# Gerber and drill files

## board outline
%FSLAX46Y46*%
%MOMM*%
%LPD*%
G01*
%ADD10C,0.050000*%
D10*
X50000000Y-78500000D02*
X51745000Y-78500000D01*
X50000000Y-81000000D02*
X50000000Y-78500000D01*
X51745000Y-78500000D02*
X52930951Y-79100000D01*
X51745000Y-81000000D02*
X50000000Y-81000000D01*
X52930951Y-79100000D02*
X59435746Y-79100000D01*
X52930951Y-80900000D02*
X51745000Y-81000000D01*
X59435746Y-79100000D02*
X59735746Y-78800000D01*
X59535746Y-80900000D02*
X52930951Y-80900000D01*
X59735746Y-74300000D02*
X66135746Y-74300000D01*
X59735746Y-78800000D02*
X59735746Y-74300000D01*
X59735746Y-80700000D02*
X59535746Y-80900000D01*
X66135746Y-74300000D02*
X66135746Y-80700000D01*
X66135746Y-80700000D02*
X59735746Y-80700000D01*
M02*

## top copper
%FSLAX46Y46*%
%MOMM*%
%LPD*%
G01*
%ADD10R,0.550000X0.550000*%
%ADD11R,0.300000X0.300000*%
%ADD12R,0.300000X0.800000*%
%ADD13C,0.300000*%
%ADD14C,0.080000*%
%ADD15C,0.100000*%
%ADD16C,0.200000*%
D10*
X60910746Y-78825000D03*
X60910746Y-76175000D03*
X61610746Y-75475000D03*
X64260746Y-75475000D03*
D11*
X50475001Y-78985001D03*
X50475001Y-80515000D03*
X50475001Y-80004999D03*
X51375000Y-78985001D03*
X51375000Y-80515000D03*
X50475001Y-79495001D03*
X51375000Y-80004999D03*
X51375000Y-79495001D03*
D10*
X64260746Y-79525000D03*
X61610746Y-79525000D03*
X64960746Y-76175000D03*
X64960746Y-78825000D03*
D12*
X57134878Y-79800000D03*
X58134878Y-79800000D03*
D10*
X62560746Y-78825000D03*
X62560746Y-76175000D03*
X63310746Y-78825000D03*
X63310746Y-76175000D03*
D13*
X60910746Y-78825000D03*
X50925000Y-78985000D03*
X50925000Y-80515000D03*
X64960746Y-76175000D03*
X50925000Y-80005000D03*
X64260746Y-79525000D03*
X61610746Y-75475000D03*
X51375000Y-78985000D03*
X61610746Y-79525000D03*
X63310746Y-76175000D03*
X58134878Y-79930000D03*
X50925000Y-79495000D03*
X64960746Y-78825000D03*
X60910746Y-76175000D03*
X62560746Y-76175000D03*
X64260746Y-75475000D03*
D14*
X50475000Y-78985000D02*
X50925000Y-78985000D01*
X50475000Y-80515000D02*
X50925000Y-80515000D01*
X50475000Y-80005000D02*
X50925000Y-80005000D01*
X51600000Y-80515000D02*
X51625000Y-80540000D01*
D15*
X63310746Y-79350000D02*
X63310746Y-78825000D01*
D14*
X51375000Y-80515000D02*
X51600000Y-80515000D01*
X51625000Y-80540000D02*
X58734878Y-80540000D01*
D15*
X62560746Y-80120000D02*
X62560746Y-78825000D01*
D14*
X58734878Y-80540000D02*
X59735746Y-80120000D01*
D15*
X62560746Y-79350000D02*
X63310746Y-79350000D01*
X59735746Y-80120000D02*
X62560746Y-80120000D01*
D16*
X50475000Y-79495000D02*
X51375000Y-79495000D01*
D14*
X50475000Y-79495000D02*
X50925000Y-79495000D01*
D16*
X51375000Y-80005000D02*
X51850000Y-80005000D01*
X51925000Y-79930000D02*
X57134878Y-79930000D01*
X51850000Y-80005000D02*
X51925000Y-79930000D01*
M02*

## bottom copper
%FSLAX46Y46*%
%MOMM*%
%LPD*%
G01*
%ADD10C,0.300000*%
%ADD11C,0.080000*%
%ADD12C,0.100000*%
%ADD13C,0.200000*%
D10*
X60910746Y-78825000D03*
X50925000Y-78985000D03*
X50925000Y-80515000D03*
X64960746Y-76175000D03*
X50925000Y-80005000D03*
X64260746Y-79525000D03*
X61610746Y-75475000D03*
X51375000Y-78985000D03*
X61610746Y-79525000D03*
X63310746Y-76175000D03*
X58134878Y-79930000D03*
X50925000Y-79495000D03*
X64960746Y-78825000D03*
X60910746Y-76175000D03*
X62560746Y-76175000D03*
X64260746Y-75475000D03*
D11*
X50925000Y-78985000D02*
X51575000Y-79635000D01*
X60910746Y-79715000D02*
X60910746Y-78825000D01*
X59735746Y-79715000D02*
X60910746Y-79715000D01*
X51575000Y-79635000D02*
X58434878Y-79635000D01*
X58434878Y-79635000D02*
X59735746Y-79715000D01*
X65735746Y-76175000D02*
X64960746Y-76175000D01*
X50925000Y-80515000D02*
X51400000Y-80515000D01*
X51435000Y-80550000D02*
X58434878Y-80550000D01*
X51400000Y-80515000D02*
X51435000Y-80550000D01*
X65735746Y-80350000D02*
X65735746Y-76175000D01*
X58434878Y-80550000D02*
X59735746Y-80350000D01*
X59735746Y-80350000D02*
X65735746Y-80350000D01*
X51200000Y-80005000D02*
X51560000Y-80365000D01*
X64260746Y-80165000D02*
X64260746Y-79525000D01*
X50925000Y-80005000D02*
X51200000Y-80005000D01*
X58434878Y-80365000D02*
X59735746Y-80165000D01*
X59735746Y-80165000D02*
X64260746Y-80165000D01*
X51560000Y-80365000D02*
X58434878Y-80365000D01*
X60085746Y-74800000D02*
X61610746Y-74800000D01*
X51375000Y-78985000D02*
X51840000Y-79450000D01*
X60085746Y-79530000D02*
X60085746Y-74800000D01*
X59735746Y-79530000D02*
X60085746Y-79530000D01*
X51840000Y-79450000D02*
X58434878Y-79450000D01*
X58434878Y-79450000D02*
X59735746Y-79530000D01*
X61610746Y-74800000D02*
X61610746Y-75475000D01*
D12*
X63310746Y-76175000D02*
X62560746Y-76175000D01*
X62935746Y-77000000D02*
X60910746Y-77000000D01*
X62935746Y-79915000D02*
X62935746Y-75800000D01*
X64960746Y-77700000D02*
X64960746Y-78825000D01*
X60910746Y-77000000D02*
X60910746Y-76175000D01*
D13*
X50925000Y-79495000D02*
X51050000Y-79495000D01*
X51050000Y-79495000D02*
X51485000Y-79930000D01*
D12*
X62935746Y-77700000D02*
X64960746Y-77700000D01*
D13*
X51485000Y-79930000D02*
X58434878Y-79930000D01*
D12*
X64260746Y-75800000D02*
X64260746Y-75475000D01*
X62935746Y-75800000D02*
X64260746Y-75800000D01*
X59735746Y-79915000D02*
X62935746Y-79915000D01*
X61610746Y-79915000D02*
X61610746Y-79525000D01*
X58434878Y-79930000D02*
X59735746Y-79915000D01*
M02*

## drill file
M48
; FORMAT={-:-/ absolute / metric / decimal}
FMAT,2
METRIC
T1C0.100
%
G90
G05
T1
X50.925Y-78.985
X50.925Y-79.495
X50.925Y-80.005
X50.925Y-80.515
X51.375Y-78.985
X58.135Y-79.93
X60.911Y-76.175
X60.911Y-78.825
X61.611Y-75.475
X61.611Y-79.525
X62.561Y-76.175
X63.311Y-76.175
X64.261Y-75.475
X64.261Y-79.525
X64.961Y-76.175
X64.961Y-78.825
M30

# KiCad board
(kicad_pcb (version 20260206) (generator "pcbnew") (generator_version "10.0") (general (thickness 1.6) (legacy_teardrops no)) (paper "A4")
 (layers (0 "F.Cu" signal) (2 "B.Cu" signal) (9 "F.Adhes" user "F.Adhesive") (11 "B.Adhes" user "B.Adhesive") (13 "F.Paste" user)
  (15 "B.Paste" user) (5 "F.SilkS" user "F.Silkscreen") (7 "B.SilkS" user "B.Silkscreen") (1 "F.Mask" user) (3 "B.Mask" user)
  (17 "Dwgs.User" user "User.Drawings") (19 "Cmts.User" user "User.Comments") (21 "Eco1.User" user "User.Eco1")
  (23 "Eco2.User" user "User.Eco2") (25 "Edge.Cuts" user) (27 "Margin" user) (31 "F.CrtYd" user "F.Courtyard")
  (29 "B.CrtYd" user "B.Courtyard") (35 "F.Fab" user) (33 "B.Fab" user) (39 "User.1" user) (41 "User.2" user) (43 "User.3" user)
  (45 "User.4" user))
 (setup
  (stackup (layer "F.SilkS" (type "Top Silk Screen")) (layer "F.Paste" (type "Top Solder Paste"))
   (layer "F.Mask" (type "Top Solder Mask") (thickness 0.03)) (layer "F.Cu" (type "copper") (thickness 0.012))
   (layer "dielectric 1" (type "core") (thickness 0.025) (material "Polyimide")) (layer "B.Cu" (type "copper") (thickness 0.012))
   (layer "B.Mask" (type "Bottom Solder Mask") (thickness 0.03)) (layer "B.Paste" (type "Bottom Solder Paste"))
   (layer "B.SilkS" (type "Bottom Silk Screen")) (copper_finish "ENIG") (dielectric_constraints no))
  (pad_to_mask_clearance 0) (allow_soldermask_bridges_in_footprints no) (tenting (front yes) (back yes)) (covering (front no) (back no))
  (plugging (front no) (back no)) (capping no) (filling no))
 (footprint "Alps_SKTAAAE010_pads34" (layer "F.Cu") (at 60.535746 77.5 90)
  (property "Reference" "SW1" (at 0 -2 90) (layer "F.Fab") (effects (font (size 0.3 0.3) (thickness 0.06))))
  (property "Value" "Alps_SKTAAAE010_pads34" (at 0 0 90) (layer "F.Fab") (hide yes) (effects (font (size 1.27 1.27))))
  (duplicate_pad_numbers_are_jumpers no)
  (pad "3" smd rect (at -1.325 0.375 90) (size 0.55 0.55) (layers "F.Cu" "F.Mask" "F.Paste") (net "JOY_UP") (solder_mask_margin 0.05)
   (thermal_bridge_angle 45))
  (pad "4" smd rect (at 1.325 0.375 90) (size 0.55 0.55) (layers "F.Cu" "F.Mask" "F.Paste") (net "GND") (solder_mask_margin 0.05)
   (thermal_bridge_angle 45)))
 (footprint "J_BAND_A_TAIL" (layer "F.Cu") (at 50.9 79.75)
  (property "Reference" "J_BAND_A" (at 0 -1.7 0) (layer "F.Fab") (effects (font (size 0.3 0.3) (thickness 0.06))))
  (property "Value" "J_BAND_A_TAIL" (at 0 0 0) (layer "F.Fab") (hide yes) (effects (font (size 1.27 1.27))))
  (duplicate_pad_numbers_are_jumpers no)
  (pad "1" smd rect (at -0.424999 -0.764999) (size 0.3 0.3) (layers "F.Cu" "F.Mask") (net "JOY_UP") (solder_mask_margin 0.05)
   (thermal_bridge_angle 45))
  (pad "2" smd rect (at -0.424999 0.765) (size 0.3 0.3) (layers "F.Cu" "F.Mask") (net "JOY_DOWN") (solder_mask_margin 0.05)
   (thermal_bridge_angle 45))
  (pad "3" smd rect (at -0.424999 0.254999) (size 0.3 0.3) (layers "F.Cu" "F.Mask") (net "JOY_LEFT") (solder_mask_margin 0.05)
   (thermal_bridge_angle 45))
  (pad "4" smd rect (at 0.475 -0.764999) (size 0.3 0.3) (layers "F.Cu" "F.Mask") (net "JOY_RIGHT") (solder_mask_margin 0.05)
   (thermal_bridge_angle 45))
  (pad "5" smd rect (at 0.475 0.765) (size 0.3 0.3) (layers "F.Cu" "F.Mask") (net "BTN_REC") (solder_mask_margin 0.05)
   (thermal_bridge_angle 45))
  (pad "6" smd rect (at -0.424999 -0.254999) (size 0.3 0.3) (layers "F.Cu" "F.Mask") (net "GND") (solder_mask_margin 0.05)
   (thermal_bridge_angle 45))
  (pad "7" smd rect (at 0.475 0.254999) (size 0.3 0.3) (layers "F.Cu" "F.Mask") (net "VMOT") (solder_mask_margin 0.05)
   (thermal_bridge_angle 45))
  (pad "8" smd rect (at 0.475 -0.254999) (size 0.3 0.3) (layers "F.Cu" "F.Mask") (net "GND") (solder_mask_margin 0.05)
   (thermal_bridge_angle 45)))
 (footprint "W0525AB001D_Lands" (layer "F.Cu") (at 57.634878 79.93)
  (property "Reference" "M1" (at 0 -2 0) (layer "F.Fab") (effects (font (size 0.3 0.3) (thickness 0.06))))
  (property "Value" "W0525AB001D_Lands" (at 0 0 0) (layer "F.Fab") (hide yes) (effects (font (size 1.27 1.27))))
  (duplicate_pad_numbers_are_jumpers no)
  (pad "1" smd rect (at -0.5 -0.13) (size 0.3 0.8) (layers "F.Cu" "F.Mask") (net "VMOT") (solder_mask_margin 0.05) (thermal_bridge_angle 45))
  (pad "2" smd rect (at 0.5 -0.13) (size 0.3 0.8) (layers "F.Cu" "F.Mask") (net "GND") (solder_mask_margin 0.05) (thermal_bridge_angle 45)))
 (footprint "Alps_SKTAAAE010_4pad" (layer "F.Cu") (at 62.935746 77.5 90)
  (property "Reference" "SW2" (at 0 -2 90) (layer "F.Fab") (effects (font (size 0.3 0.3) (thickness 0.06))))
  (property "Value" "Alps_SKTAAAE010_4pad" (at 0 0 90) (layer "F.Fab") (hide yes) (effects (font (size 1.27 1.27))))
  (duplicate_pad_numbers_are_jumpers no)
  (pad "1" smd rect (at -1.325 -0.375 90) (size 0.55 0.55) (layers "F.Cu" "F.Mask" "F.Paste") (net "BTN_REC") (solder_mask_margin 0.05)
   (thermal_bridge_angle 45))
  (pad "2" smd rect (at 1.325 -0.375 90) (size 0.55 0.55) (layers "F.Cu" "F.Mask" "F.Paste") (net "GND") (solder_mask_margin 0.05)
   (thermal_bridge_angle 45))
  (pad "3" smd rect (at -1.325 0.375 90) (size 0.55 0.55) (layers "F.Cu" "F.Mask" "F.Paste") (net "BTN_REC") (solder_mask_margin 0.05)
   (thermal_bridge_angle 45))
  (pad "4" smd rect (at 1.325 0.375 90) (size 0.55 0.55) (layers "F.Cu" "F.Mask" "F.Paste") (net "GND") (solder_mask_margin 0.05)
   (thermal_bridge_angle 45)))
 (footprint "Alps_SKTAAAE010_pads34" (layer "F.Cu") (at 62.935746 79.9 180)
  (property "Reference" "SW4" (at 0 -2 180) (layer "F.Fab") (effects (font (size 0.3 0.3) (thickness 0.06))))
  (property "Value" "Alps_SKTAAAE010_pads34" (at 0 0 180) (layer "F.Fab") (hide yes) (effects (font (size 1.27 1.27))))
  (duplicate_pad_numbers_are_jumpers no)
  (pad "3" smd rect (at -1.325 0.375 180) (size 0.55 0.55) (layers "F.Cu" "F.Mask" "F.Paste") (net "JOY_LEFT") (solder_mask_margin 0.05)
   (thermal_bridge_angle 45))
  (pad "4" smd rect (at 1.325 0.375 180) (size 0.55 0.55) (layers "F.Cu" "F.Mask" "F.Paste") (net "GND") (solder_mask_margin 0.05)
   (thermal_bridge_angle 45)))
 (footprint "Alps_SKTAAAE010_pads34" (layer "F.Cu") (at 65.335746 77.5 -90)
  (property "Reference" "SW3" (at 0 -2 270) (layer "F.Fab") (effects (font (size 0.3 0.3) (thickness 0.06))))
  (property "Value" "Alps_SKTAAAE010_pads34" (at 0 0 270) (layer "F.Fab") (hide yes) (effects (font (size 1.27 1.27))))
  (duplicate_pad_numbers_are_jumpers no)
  (pad "3" smd rect (at -1.325 0.375 270) (size 0.55 0.55) (layers "F.Cu" "F.Mask" "F.Paste") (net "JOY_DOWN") (solder_mask_margin 0.05)
   (thermal_bridge_angle 45))
  (pad "4" smd rect (at 1.325 0.375 270) (size 0.55 0.55) (layers "F.Cu" "F.Mask" "F.Paste") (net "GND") (solder_mask_margin 0.05)
   (thermal_bridge_angle 45)))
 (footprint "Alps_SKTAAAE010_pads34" (layer "F.Cu") (at 62.935746 75.1)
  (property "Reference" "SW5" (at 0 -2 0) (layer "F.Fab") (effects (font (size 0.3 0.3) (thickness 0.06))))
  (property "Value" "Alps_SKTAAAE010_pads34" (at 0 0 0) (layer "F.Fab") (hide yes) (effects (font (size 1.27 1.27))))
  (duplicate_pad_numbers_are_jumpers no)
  (pad "3" smd rect (at -1.325 0.375) (size 0.55 0.55) (layers "F.Cu" "F.Mask" "F.Paste") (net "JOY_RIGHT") (solder_mask_margin 0.05)
   (thermal_bridge_angle 45))
  (pad "4" smd rect (at 1.325 0.375) (size 0.55 0.55) (layers "F.Cu" "F.Mask" "F.Paste") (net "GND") (solder_mask_margin 0.05)
   (thermal_bridge_angle 45)))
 (gr_line (start 50 78.5) (end 51.745 78.5) (stroke (width 0.05) (type default)) (layer "Edge.Cuts"))
 (gr_line (start 50 81) (end 50 78.5) (stroke (width 0.05) (type default)) (layer "Edge.Cuts"))
 (gr_line (start 51.745 78.5) (end 52.930951 79.1) (stroke (width 0.05) (type default)) (layer "Edge.Cuts"))
 (gr_line (start 51.745 81) (end 50 81) (stroke (width 0.05) (type default)) (layer "Edge.Cuts"))
 (gr_line (start 52.930951 79.1) (end 59.435746 79.1) (stroke (width 0.05) (type default)) (layer "Edge.Cuts"))
 (gr_line (start 52.930951 80.9) (end 51.745 81) (stroke (width 0.05) (type default)) (layer "Edge.Cuts"))
 (gr_line (start 59.435746 79.1) (end 59.735746 78.8) (stroke (width 0.05) (type default)) (layer "Edge.Cuts"))
 (gr_line (start 59.535746 80.9) (end 52.930951 80.9) (stroke (width 0.05) (type default)) (layer "Edge.Cuts"))
 (gr_line (start 59.735746 74.3) (end 66.135746 74.3) (stroke (width 0.05) (type default)) (layer "Edge.Cuts"))
 (gr_line (start 59.735746 78.8) (end 59.735746 74.3) (stroke (width 0.05) (type default)) (layer "Edge.Cuts"))
 (gr_line (start 59.735746 80.7) (end 59.535746 80.9) (stroke (width 0.05) (type default)) (layer "Edge.Cuts"))
 (gr_line (start 66.135746 74.3) (end 66.135746 80.7) (stroke (width 0.05) (type default)) (layer "Edge.Cuts"))
 (gr_line (start 66.135746 80.7) (end 59.735746 80.7) (stroke (width 0.05) (type default)) (layer "Edge.Cuts"))
 (segment (start 50.475 78.985) (end 50.925 78.985) (width 0.08) (layer "F.Cu") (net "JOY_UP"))
 (via (at 50.925 78.985) (size 0.3) (drill 0.1) (layers "F.Cu" "B.Cu") (tenting (front yes) (back yes)) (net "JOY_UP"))
 (via (at 60.910746 78.825) (size 0.3) (drill 0.1) (layers "F.Cu" "B.Cu") (tenting (front yes) (back yes)) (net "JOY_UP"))
 (segment (start 50.925 78.985) (end 51.575 79.635) (width 0.08) (layer "B.Cu") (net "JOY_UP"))
 (segment (start 60.910746 79.715) (end 60.910746 78.825) (width 0.08) (layer "B.Cu") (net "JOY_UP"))
 (segment (start 59.735746 79.715) (end 60.910746 79.715) (width 0.08) (layer "B.Cu") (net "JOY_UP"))
 (segment (start 51.575 79.635) (end 58.434878 79.635) (width 0.08) (layer "B.Cu") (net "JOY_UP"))
 (segment (start 58.434878 79.635) (end 59.735746 79.715) (width 0.08) (layer "B.Cu") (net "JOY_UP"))
 (segment (start 50.475 80.515) (end 50.925 80.515) (width 0.08) (layer "F.Cu") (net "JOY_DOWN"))
 (via (at 50.925 80.515) (size 0.3) (drill 0.1) (layers "F.Cu" "B.Cu") (tenting (front yes) (back yes)) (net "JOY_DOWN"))
 (via (at 64.960746 76.175) (size 0.3) (drill 0.1) (layers "F.Cu" "B.Cu") (tenting (front yes) (back yes)) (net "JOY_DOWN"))
 (segment (start 59.735746 80.35) (end 65.735746 80.35) (width 0.08) (layer "B.Cu") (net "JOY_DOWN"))
 (segment (start 51.4 80.515) (end 51.435 80.55) (width 0.08) (layer "B.Cu") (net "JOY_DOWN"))
 (segment (start 65.735746 76.175) (end 64.960746 76.175) (width 0.08) (layer "B.Cu") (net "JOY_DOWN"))
 (segment (start 50.925 80.515) (end 51.4 80.515) (width 0.08) (layer "B.Cu") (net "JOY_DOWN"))
 (segment (start 51.435 80.55) (end 58.434878 80.55) (width 0.08) (layer "B.Cu") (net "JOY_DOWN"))
 (segment (start 58.434878 80.55) (end 59.735746 80.35) (width 0.08) (layer "B.Cu") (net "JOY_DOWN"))
 (segment (start 65.735746 80.35) (end 65.735746 76.175) (width 0.08) (layer "B.Cu") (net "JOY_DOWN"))
 (segment (start 50.475 80.005) (end 50.925 80.005) (width 0.08) (layer "F.Cu") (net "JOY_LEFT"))
 (via (at 64.260746 79.525) (size 0.3) (drill 0.1) (layers "F.Cu" "B.Cu") (tenting (front yes) (back yes)) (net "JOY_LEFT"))
 (via (at 50.925 80.005) (size 0.3) (drill 0.1) (layers "F.Cu" "B.Cu") (tenting (front yes) (back yes)) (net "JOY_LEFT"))
 (segment (start 50.925 80.005) (end 51.2 80.005) (width 0.08) (layer "B.Cu") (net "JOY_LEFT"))
 (segment (start 51.56 80.365) (end 58.434878 80.365) (width 0.08) (layer "B.Cu") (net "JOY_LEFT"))
 (segment (start 58.434878 80.365) (end 59.735746 80.165) (width 0.08) (layer "B.Cu") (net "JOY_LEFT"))
 (segment (start 51.2 80.005) (end 51.56 80.365) (width 0.08) (layer "B.Cu") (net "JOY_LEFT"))
 (segment (start 59.735746 80.165) (end 64.260746 80.165) (width 0.08) (layer "B.Cu") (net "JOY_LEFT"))
 (segment (start 64.260746 80.165) (end 64.260746 79.525) (width 0.08) (layer "B.Cu") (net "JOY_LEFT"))
 (via (at 51.375 78.985) (size 0.3) (drill 0.1) (layers "F.Cu" "B.Cu") (tenting (front yes) (back yes)) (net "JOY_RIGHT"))
 (via (at 61.610746 75.475) (size 0.3) (drill 0.1) (layers "F.Cu" "B.Cu") (tenting (front yes) (back yes)) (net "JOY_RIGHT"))
 (segment (start 60.085746 79.53) (end 60.085746 74.8) (width 0.08) (layer "B.Cu") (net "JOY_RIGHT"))
 (segment (start 51.375 78.985) (end 51.84 79.45) (width 0.08) (layer "B.Cu") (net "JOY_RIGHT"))
 (segment (start 61.610746 74.8) (end 61.610746 75.475) (width 0.08) (layer "B.Cu") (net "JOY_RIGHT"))
 (segment (start 51.84 79.45) (end 58.434878 79.45) (width 0.08) (layer "B.Cu") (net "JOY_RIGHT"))
 (segment (start 58.434878 79.45) (end 59.735746 79.53) (width 0.08) (layer "B.Cu") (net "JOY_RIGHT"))
 (segment (start 59.735746 79.53) (end 60.085746 79.53) (width 0.08) (layer "B.Cu") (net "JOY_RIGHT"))
 (segment (start 60.085746 74.8) (end 61.610746 74.8) (width 0.08) (layer "B.Cu") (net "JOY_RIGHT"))
 (segment (start 51.375 80.515) (end 51.6 80.515) (width 0.08) (layer "F.Cu") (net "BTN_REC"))
 (segment (start 62.560746 79.35) (end 63.310746 79.35) (width 0.1) (layer "F.Cu") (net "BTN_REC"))
 (segment (start 51.6 80.515) (end 51.625 80.54) (width 0.08) (layer "F.Cu") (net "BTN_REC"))
 (segment (start 58.734878 80.54) (end 59.735746 80.12) (width 0.08) (layer "F.Cu") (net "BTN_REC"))
 (segment (start 59.735746 80.12) (end 62.560746 80.12) (width 0.1) (layer "F.Cu") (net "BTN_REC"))
 (segment (start 62.560746 80.12) (end 62.560746 78.825) (width 0.1) (layer "F.Cu") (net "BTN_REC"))
 (segment (start 51.625 80.54) (end 58.734878 80.54) (width 0.08) (layer "F.Cu") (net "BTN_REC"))
 (segment (start 63.310746 79.35) (end 63.310746 78.825) (width 0.1) (layer "F.Cu") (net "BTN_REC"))
 (segment (start 50.475 79.495) (end 51.375 79.495) (width 0.2) (layer "F.Cu") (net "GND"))
 (segment (start 50.475 79.495) (end 50.925 79.495) (width 0.08) (layer "F.Cu") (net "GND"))
 (via (at 63.310746 76.175) (size 0.3) (drill 0.1) (layers "F.Cu" "B.Cu") (tenting (front yes) (back yes)) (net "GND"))
 (via (at 64.260746 75.475) (size 0.3) (drill 0.1) (layers "F.Cu" "B.Cu") (tenting (front yes) (back yes)) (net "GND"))
 (via (at 61.610746 79.525) (size 0.3) (drill 0.1) (layers "F.Cu" "B.Cu") (tenting (front yes) (back yes)) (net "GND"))
 (via (at 60.910746 76.175) (size 0.3) (drill 0.1) (layers "F.Cu" "B.Cu") (tenting (front yes) (back yes)) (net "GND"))
 (via (at 62.560746 76.175) (size 0.3) (drill 0.1) (layers "F.Cu" "B.Cu") (tenting (front yes) (back yes)) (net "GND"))
 (via (at 50.925 79.495) (size 0.3) (drill 0.1) (layers "F.Cu" "B.Cu") (tenting (front yes) (back yes)) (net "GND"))
 (via (at 58.134878 79.93) (size 0.3) (drill 0.1) (layers "F.Cu" "B.Cu") (tenting (front yes) (back yes)) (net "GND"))
 (via (at 64.960746 78.825) (size 0.3) (drill 0.1) (layers "F.Cu" "B.Cu") (tenting (front yes) (back yes)) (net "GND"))
 (segment (start 64.960746 77.7) (end 64.960746 78.825) (width 0.1) (layer "B.Cu") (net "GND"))
 (segment (start 58.434878 79.93) (end 59.735746 79.915) (width 0.1) (layer "B.Cu") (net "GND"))
 (segment (start 62.935746 77) (end 60.910746 77) (width 0.1) (layer "B.Cu") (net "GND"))
 (segment (start 50.925 79.495) (end 51.05 79.495) (width 0.2) (layer "B.Cu") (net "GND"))
 (segment (start 62.935746 77.7) (end 64.960746 77.7) (width 0.1) (layer "B.Cu") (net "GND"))
 (segment (start 60.910746 77) (end 60.910746 76.175) (width 0.1) (layer "B.Cu") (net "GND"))
 (segment (start 62.935746 79.915) (end 62.935746 75.8) (width 0.1) (layer "B.Cu") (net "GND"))
 (segment (start 63.310746 76.175) (end 62.560746 76.175) (width 0.1) (layer "B.Cu") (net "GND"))
 (segment (start 59.735746 79.915) (end 62.935746 79.915) (width 0.1) (layer "B.Cu") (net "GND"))
 (segment (start 51.05 79.495) (end 51.485 79.93) (width 0.2) (layer "B.Cu") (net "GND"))
 (segment (start 64.260746 75.8) (end 64.260746 75.475) (width 0.1) (layer "B.Cu") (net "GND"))
 (segment (start 61.610746 79.915) (end 61.610746 79.525) (width 0.1) (layer "B.Cu") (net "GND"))
 (segment (start 51.485 79.93) (end 58.434878 79.93) (width 0.2) (layer "B.Cu") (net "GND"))
 (segment (start 62.935746 75.8) (end 64.260746 75.8) (width 0.1) (layer "B.Cu") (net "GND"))
 (segment (start 51.925 79.93) (end 57.134878 79.93) (width 0.2) (layer "F.Cu") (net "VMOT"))
 (segment (start 51.85 80.005) (end 51.925 79.93) (width 0.2) (layer "F.Cu") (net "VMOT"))
 (segment (start 51.375 80.005) (end 51.85 80.005) (width 0.2) (layer "F.Cu") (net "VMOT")))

